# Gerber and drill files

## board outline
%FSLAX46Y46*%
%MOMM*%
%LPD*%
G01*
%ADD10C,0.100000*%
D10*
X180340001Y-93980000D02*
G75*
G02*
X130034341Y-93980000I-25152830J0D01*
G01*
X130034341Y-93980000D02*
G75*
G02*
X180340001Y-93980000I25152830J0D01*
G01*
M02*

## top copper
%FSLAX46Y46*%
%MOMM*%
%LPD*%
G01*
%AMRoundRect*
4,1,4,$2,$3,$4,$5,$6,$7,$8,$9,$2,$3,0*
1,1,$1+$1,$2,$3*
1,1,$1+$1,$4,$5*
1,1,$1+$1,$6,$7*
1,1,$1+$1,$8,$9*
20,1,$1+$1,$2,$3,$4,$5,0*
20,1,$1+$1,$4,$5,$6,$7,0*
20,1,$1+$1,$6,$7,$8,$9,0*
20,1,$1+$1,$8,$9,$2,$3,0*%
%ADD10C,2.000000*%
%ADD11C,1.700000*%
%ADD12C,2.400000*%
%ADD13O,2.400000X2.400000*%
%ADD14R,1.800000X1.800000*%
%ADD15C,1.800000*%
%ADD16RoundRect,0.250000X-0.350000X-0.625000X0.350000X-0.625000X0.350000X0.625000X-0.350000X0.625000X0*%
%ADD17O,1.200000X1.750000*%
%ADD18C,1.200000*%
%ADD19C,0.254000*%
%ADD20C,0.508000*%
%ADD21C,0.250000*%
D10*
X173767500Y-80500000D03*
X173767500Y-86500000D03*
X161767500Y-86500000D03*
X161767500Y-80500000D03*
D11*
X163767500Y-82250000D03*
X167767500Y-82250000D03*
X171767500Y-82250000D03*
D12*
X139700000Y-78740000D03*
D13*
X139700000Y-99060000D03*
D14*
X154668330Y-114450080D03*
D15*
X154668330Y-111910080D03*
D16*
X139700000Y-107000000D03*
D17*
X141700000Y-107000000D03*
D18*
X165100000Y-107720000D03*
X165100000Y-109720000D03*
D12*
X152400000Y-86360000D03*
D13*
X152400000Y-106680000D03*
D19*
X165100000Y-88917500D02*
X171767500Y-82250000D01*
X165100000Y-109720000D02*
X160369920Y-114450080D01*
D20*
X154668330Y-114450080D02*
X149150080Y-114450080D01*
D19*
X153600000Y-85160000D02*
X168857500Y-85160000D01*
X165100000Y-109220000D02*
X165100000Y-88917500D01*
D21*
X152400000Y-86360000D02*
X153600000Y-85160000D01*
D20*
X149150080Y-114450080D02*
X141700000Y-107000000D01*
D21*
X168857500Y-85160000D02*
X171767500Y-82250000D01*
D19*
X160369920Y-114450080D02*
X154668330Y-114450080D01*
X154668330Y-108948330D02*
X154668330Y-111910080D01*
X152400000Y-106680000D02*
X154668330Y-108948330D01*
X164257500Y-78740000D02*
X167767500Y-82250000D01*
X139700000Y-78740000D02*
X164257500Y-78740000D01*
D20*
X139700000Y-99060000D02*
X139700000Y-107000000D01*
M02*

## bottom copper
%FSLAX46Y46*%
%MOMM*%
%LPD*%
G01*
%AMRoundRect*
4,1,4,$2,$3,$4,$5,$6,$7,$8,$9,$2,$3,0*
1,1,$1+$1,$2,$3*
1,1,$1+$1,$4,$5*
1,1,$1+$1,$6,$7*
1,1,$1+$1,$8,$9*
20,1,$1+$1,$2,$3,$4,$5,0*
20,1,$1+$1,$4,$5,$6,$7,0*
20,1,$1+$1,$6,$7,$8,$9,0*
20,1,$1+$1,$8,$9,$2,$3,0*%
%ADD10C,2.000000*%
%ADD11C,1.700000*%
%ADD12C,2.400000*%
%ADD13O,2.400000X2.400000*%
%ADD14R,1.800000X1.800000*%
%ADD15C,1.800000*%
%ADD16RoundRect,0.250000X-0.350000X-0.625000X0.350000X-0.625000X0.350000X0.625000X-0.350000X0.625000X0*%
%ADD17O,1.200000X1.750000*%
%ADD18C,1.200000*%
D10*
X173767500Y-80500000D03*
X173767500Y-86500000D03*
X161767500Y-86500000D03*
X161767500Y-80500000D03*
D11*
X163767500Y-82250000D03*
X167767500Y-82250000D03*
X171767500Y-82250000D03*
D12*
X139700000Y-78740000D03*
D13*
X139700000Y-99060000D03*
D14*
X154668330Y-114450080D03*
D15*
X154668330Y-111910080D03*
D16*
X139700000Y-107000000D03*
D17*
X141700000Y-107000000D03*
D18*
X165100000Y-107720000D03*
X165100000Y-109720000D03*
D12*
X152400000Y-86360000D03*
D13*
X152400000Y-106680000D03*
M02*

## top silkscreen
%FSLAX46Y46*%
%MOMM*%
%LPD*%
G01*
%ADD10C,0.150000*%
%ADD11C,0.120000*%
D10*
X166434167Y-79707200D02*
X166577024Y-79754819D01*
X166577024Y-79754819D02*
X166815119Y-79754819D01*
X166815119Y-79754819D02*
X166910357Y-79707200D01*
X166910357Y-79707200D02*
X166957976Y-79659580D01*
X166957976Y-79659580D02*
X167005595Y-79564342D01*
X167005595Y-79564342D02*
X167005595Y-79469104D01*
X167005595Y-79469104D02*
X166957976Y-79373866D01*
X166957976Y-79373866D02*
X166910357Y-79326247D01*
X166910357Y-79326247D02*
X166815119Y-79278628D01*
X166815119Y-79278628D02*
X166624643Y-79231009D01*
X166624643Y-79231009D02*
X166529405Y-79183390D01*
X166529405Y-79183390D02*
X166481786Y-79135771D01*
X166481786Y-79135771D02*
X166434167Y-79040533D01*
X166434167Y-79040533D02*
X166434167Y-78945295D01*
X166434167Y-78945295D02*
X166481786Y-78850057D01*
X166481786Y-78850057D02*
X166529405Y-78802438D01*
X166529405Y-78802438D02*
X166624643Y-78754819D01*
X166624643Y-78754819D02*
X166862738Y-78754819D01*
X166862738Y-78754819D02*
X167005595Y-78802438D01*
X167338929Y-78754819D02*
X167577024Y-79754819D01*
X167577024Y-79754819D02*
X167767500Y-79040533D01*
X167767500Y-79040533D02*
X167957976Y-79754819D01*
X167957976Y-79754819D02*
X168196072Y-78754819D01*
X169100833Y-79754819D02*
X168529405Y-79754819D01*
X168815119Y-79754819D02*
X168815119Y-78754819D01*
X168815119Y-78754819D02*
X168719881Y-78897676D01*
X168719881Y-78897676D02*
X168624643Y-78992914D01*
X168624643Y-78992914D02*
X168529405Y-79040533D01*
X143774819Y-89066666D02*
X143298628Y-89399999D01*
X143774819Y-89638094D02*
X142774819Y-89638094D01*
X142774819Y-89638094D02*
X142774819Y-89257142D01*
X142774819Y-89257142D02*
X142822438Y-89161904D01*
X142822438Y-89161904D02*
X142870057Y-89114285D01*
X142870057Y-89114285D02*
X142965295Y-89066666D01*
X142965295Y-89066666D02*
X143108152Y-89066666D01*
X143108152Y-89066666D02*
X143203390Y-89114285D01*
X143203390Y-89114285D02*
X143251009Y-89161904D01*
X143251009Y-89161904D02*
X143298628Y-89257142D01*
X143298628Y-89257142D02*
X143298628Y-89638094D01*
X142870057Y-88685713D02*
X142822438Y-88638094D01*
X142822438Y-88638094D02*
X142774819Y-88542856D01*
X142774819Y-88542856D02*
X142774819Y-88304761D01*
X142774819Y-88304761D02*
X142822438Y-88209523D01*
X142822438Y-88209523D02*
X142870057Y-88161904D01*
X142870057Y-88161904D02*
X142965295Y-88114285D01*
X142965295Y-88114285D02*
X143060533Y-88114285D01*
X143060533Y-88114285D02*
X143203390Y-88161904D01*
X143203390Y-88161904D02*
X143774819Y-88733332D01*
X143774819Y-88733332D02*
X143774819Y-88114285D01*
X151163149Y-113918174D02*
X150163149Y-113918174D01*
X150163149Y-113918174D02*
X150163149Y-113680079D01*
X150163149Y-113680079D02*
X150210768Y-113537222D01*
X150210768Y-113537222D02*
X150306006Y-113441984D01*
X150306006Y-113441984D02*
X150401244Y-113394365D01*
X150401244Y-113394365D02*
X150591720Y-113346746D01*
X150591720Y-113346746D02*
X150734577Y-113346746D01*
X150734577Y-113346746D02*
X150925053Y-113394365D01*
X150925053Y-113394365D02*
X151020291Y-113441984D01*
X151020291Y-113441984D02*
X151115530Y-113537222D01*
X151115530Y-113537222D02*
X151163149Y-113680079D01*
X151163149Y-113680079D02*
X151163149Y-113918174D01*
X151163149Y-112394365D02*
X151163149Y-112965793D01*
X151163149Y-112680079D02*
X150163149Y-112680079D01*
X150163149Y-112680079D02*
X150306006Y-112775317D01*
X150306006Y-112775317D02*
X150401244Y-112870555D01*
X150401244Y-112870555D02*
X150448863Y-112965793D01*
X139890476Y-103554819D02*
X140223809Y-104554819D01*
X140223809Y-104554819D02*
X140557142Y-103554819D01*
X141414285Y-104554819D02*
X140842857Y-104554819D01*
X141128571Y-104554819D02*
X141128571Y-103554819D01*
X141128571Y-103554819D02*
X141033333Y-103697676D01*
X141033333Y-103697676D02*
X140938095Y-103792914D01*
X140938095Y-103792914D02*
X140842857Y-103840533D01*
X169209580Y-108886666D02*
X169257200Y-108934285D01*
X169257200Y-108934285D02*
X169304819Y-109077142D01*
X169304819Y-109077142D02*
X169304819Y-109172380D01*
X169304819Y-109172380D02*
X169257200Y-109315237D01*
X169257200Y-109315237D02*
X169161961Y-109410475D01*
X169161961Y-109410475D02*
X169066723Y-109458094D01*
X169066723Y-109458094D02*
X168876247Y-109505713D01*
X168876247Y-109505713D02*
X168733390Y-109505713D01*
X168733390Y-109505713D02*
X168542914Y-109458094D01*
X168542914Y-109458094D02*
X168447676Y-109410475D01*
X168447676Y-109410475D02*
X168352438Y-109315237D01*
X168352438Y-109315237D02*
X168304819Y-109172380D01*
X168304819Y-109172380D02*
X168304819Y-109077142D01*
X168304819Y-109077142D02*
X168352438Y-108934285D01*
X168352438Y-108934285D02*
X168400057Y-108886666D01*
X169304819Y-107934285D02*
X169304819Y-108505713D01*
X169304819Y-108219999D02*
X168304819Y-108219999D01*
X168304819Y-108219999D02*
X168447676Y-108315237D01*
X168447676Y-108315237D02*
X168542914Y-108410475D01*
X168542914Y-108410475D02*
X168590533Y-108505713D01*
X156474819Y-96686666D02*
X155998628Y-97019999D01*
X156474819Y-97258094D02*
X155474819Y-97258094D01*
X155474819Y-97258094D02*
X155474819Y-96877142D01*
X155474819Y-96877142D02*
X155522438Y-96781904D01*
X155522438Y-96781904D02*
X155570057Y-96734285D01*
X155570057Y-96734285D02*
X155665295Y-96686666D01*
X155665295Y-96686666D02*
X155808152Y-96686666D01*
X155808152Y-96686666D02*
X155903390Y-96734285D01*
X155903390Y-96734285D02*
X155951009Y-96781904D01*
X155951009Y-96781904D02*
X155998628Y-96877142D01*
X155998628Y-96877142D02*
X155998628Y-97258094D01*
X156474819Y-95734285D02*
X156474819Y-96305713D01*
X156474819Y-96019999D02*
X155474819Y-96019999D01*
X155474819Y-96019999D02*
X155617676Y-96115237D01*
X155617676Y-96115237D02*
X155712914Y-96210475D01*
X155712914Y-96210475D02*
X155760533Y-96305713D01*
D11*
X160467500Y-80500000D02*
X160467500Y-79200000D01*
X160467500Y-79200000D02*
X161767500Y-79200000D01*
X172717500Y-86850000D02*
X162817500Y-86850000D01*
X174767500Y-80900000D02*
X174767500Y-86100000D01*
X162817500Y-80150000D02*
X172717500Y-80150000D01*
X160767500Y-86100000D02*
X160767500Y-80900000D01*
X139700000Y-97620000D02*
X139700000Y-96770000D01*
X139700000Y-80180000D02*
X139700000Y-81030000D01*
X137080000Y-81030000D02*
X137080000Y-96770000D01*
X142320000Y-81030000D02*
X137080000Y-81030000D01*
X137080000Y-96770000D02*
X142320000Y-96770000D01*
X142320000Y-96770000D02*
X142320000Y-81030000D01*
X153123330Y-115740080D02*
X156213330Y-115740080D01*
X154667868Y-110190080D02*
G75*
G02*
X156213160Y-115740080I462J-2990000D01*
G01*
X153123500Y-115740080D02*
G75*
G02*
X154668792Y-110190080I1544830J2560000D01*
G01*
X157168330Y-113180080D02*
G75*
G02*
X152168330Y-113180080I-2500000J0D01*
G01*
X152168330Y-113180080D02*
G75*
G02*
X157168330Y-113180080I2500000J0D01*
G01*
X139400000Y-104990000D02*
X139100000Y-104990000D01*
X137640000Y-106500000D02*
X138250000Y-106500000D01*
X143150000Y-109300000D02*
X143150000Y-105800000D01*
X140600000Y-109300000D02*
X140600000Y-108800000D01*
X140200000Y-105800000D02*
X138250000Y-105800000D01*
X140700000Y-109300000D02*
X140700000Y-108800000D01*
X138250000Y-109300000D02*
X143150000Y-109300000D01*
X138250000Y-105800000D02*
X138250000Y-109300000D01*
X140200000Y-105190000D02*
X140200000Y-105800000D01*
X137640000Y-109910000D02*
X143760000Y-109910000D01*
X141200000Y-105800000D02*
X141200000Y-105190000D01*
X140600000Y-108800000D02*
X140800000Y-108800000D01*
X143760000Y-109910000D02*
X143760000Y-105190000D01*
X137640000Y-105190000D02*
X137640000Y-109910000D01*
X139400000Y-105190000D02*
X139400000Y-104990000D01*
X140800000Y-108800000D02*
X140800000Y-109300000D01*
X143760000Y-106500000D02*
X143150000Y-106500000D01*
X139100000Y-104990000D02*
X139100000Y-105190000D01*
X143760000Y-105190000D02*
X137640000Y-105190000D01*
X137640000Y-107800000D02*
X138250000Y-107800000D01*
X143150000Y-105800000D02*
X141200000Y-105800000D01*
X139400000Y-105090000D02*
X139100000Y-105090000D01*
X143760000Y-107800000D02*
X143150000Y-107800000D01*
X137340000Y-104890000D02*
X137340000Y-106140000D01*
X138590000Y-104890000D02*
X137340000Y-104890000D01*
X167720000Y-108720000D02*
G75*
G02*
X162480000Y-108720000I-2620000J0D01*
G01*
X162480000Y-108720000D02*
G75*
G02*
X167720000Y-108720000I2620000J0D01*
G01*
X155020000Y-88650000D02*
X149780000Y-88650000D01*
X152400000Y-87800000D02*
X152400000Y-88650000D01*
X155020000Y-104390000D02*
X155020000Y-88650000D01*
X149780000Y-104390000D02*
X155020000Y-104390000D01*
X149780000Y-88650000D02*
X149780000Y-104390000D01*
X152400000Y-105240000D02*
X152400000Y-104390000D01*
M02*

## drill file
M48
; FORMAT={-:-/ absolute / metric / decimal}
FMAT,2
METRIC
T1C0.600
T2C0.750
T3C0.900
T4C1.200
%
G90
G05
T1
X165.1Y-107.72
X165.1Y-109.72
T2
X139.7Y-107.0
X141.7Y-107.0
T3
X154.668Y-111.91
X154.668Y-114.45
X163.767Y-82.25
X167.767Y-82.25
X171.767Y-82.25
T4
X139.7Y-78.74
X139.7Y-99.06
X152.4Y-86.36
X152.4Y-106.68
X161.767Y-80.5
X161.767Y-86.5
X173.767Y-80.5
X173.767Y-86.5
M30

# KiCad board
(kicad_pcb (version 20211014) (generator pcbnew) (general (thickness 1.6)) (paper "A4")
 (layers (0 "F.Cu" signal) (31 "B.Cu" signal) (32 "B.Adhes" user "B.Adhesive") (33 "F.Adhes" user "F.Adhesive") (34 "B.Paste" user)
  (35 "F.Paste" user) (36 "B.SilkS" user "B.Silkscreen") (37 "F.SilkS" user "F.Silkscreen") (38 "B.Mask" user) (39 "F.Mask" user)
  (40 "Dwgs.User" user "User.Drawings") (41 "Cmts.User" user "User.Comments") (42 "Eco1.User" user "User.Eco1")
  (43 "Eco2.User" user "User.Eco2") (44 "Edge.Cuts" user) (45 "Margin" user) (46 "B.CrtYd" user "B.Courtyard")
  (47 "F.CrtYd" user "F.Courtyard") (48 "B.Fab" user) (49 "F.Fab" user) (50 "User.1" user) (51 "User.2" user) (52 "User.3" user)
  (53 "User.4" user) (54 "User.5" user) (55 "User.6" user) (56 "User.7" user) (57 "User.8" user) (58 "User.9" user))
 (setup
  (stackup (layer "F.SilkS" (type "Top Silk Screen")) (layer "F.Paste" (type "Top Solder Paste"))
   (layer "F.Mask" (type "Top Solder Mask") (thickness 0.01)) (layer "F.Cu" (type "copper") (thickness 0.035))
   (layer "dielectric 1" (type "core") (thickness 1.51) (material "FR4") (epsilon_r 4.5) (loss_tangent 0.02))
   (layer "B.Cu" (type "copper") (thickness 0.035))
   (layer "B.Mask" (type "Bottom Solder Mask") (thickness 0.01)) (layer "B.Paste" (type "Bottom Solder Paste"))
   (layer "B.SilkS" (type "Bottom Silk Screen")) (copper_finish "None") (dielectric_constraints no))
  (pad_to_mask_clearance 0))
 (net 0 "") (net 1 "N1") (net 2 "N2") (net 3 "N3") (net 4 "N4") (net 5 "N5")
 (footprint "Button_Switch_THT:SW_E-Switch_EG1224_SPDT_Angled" (layer "F.Cu") (at 163.7675 82.25)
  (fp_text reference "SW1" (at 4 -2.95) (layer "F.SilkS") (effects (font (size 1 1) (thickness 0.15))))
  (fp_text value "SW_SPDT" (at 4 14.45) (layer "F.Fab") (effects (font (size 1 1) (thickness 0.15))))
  (fp_line (start -3.3 -1.75) (end -3.3 -3.05) (layer "F.SilkS") (width 0.12))
  (fp_line (start -3.3 -3.05) (end -2 -3.05) (layer "F.SilkS") (width 0.12))
  (fp_line (start 8.95 4.6) (end -0.95 4.6) (layer "F.SilkS") (width 0.12))
  (fp_line (start 11 -1.35) (end 11 3.85) (layer "F.SilkS") (width 0.12))
  (fp_line (start -0.95 -2.1) (end 8.95 -2.1) (layer "F.SilkS") (width 0.12))
  (fp_line (start -3 3.85) (end -3 -1.35) (layer "F.SilkS") (width 0.12))
  (pad "" thru_hole circle (at 10 -1.75) (size 2 2) (drill 1.2) (layers *.Cu *.Mask))
  (pad "" thru_hole circle (at 10 4.25) (size 2 2) (drill 1.2) (layers *.Cu *.Mask))
  (pad "" thru_hole circle (at -2 4.25) (size 2 2) (drill 1.2) (layers *.Cu *.Mask))
  (pad "" thru_hole circle (at -2 -1.75) (size 2 2) (drill 1.2) (layers *.Cu *.Mask))
  (pad "1" thru_hole circle (at 0 0) (size 1.7 1.7) (drill 0.9) (layers *.Cu *.Mask) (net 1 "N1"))
  (pad "2" thru_hole circle (at 4 0) (size 1.7 1.7) (drill 0.9) (layers *.Cu *.Mask) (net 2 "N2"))
  (pad "3" thru_hole circle (at 8 0) (size 1.7 1.7) (drill 0.9) (layers *.Cu *.Mask) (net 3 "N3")))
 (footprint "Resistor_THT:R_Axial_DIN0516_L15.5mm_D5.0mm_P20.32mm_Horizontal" (layer "F.Cu") (at 139.7 78.74 -90)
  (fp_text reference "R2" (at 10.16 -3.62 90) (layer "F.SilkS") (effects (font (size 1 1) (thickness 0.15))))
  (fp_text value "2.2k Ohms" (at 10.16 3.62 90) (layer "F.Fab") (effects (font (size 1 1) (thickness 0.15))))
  (fp_line (start 18.88 0) (end 18.03 0) (layer "F.SilkS") (width 0.12))
  (fp_line (start 1.44 0) (end 2.29 0) (layer "F.SilkS") (width 0.12))
  (fp_line (start 2.29 2.62) (end 18.03 2.62) (layer "F.SilkS") (width 0.12))
  (fp_line (start 2.29 -2.62) (end 2.29 2.62) (layer "F.SilkS") (width 0.12))
  (fp_line (start 18.03 2.62) (end 18.03 -2.62) (layer "F.SilkS") (width 0.12))
  (fp_line (start 18.03 -2.62) (end 2.29 -2.62) (layer "F.SilkS") (width 0.12))
  (pad "1" thru_hole circle (at 0 0 270) (size 2.4 2.4) (drill 1.2) (layers *.Cu *.Mask) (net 2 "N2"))
  (pad "2" thru_hole oval (at 20.32 0 270) (size 2.4 2.4) (drill 1.2) (layers *.Cu *.Mask) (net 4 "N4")))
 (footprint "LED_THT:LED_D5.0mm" (layer "F.Cu") (at 154.66833 114.45008 90)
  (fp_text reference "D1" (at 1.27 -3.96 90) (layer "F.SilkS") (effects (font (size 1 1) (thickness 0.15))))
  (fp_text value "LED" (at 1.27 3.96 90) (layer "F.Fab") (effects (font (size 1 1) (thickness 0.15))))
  (fp_line (start -1.29 -1.545) (end -1.29 1.545) (layer "F.SilkS") (width 0.12))
  (fp_arc (start 4.26 -0.000462) (mid 2.072002 2.880433) (end -1.29 1.54483) (layer "F.SilkS") (width 0.12))
  (fp_arc (start -1.29 -1.54483) (mid 2.072002 -2.880433) (end 4.26 0.000462) (layer "F.SilkS") (width 0.12))
  (fp_circle (center 1.27 0) (end 3.77 0) (layer "F.SilkS") (width 0.12) (fill none))
  (pad "1" thru_hole rect (at 0 0 90) (size 1.8 1.8) (drill 0.9) (layers *.Cu *.Mask) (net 3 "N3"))
  (pad "2" thru_hole circle (at 2.54 0 90) (size 1.8 1.8) (drill 0.9) (layers *.Cu *.Mask) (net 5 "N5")))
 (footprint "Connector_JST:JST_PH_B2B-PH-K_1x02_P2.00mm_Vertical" (layer "F.Cu") (at 139.7 107)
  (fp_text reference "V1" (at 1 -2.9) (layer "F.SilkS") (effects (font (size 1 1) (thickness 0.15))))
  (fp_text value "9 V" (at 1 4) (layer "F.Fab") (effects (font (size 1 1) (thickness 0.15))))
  (fp_line (start -0.3 -2.01) (end -0.6 -2.01) (layer "F.SilkS") (width 0.12))
  (fp_line (start -2.06 -0.5) (end -1.45 -0.5) (layer "F.SilkS") (width 0.12))
  (fp_line (start 3.45 2.3) (end 3.45 -1.2) (layer "F.SilkS") (width 0.12))
  (fp_line (start 0.9 2.3) (end 0.9 1.8) (layer "F.SilkS") (width 0.12))
  (fp_line (start 0.5 -1.2) (end -1.45 -1.2) (layer "F.SilkS") (width 0.12))
  (fp_line (start 1 2.3) (end 1 1.8) (layer "F.SilkS") (width 0.12))
  (fp_line (start -1.45 2.3) (end 3.45 2.3) (layer "F.SilkS") (width 0.12))
  (fp_line (start -1.45 -1.2) (end -1.45 2.3) (layer "F.SilkS") (width 0.12))
  (fp_line (start 0.5 -1.81) (end 0.5 -1.2) (layer "F.SilkS") (width 0.12))
  (fp_line (start -2.06 2.91) (end 4.06 2.91) (layer "F.SilkS") (width 0.12))
  (fp_line (start 1.5 -1.2) (end 1.5 -1.81) (layer "F.SilkS") (width 0.12))
  (fp_line (start 0.9 1.8) (end 1.1 1.8) (layer "F.SilkS") (width 0.12))
  (fp_line (start 4.06 2.91) (end 4.06 -1.81) (layer "F.SilkS") (width 0.12))
  (fp_line (start -2.06 -1.81) (end -2.06 2.91) (layer "F.SilkS") (width 0.12))
  (fp_line (start -0.3 -1.81) (end -0.3 -2.01) (layer "F.SilkS") (width 0.12))
  (fp_line (start 1.1 1.8) (end 1.1 2.3) (layer "F.SilkS") (width 0.12))
  (fp_line (start 4.06 -0.5) (end 3.45 -0.5) (layer "F.SilkS") (width 0.12))
  (fp_line (start -0.6 -2.01) (end -0.6 -1.81) (layer "F.SilkS") (width 0.12))
  (fp_line (start 4.06 -1.81) (end -2.06 -1.81) (layer "F.SilkS") (width 0.12))
  (fp_line (start -2.06 0.8) (end -1.45 0.8) (layer "F.SilkS") (width 0.12))
  (fp_line (start 3.45 -1.2) (end 1.5 -1.2) (layer "F.SilkS") (width 0.12))
  (fp_line (start -0.3 -1.91) (end -0.6 -1.91) (layer "F.SilkS") (width 0.12))
  (fp_line (start 4.06 0.8) (end 3.45 0.8) (layer "F.SilkS") (width 0.12))
  (fp_line (start -2.36 -2.11) (end -2.36 -0.86) (layer "F.SilkS") (width 0.12))
  (fp_line (start -1.11 -2.11) (end -2.36 -2.11) (layer "F.SilkS") (width 0.12))
  (pad "1" thru_hole roundrect (at 0 0) (size 1.2 1.75) (drill 0.75) (layers *.Cu *.Mask) (roundrect_rratio 0.208333) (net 4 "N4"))
  (pad "2" thru_hole oval (at 2 0) (size 1.2 1.75) (drill 0.75) (layers *.Cu *.Mask) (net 3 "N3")))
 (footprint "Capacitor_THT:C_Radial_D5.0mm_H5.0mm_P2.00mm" (layer "F.Cu") (at 165.1 107.72 -90)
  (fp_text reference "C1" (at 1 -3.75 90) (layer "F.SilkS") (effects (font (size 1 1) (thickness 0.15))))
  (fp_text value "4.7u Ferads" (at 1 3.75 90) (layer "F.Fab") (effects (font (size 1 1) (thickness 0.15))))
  (fp_circle (center 1 0) (end 3.62 0) (layer "F.SilkS") (width 0.12) (fill none))
  (pad "1" thru_hole circle (at 0 0 270) (size 1.2 1.2) (drill 0.6) (layers *.Cu *.Mask) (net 3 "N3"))
  (pad "2" thru_hole circle (at 2 0 270) (size 1.2 1.2) (drill 0.6) (layers *.Cu *.Mask) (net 3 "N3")))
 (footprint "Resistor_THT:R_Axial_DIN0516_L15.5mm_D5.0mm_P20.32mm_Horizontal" (layer "F.Cu") (at 152.4 86.36 -90)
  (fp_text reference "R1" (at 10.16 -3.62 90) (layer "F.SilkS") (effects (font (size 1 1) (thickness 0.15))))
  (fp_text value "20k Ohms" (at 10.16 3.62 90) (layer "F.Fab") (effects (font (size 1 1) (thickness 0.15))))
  (fp_line (start 2.29 -2.62) (end 2.29 2.62) (layer "F.SilkS") (width 0.12))
  (fp_line (start 1.44 0) (end 2.29 0) (layer "F.SilkS") (width 0.12))
  (fp_line (start 18.03 -2.62) (end 2.29 -2.62) (layer "F.SilkS") (width 0.12))
  (fp_line (start 18.03 2.62) (end 18.03 -2.62) (layer "F.SilkS") (width 0.12))
  (fp_line (start 2.29 2.62) (end 18.03 2.62) (layer "F.SilkS") (width 0.12))
  (fp_line (start 18.88 0) (end 18.03 0) (layer "F.SilkS") (width 0.12))
  (pad "1" thru_hole circle (at 0 0 270) (size 2.4 2.4) (drill 1.2) (layers *.Cu *.Mask) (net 3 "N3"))
  (pad "2" thru_hole oval (at 20.32 0 270) (size 2.4 2.4) (drill 1.2) (layers *.Cu *.Mask) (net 5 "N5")))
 (gr_circle (center 155.187171 93.98) (end 178.196718 104.14) (layer "Edge.Cuts") (width 0.1) (fill none))
 (segment (start 165.1 88.9175) (end 171.7675 82.25) (width 0.254) (layer "F.Cu") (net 3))
 (segment (start 165.1 109.72) (end 160.36992 114.45008) (width 0.254) (layer "F.Cu") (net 3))
 (segment (start 154.66833 114.45008) (end 149.15008 114.45008) (width 0.508) (layer "F.Cu") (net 3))
 (segment (start 153.6 85.16) (end 168.8575 85.16) (width 0.254) (layer "F.Cu") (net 3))
 (segment (start 165.1 109.22) (end 165.1 88.9175) (width 0.254) (layer "F.Cu") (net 3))
 (segment (start 152.4 86.36) (end 153.6 85.16) (width 0.25) (layer "F.Cu") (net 3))
 (segment (start 149.15008 114.45008) (end 141.7 107) (width 0.508) (layer "F.Cu") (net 3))
 (segment (start 168.8575 85.16) (end 171.7675 82.25) (width 0.25) (layer "F.Cu") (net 3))
 (segment (start 160.36992 114.45008) (end 154.66833 114.45008) (width 0.254) (layer "F.Cu") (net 3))
 (segment (start 154.66833 108.94833) (end 154.66833 111.91008) (width 0.254) (layer "F.Cu") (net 5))
 (segment (start 152.4 106.68) (end 154.66833 108.94833) (width 0.254) (layer "F.Cu") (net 5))
 (segment (start 164.2575 78.74) (end 167.7675 82.25) (width 0.254) (layer "F.Cu") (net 2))
 (segment (start 139.7 78.74) (end 164.2575 78.74) (width 0.254) (layer "F.Cu") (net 2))
 (segment (start 139.7 99.06) (end 139.7 107) (width 0.508) (layer "F.Cu") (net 4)))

